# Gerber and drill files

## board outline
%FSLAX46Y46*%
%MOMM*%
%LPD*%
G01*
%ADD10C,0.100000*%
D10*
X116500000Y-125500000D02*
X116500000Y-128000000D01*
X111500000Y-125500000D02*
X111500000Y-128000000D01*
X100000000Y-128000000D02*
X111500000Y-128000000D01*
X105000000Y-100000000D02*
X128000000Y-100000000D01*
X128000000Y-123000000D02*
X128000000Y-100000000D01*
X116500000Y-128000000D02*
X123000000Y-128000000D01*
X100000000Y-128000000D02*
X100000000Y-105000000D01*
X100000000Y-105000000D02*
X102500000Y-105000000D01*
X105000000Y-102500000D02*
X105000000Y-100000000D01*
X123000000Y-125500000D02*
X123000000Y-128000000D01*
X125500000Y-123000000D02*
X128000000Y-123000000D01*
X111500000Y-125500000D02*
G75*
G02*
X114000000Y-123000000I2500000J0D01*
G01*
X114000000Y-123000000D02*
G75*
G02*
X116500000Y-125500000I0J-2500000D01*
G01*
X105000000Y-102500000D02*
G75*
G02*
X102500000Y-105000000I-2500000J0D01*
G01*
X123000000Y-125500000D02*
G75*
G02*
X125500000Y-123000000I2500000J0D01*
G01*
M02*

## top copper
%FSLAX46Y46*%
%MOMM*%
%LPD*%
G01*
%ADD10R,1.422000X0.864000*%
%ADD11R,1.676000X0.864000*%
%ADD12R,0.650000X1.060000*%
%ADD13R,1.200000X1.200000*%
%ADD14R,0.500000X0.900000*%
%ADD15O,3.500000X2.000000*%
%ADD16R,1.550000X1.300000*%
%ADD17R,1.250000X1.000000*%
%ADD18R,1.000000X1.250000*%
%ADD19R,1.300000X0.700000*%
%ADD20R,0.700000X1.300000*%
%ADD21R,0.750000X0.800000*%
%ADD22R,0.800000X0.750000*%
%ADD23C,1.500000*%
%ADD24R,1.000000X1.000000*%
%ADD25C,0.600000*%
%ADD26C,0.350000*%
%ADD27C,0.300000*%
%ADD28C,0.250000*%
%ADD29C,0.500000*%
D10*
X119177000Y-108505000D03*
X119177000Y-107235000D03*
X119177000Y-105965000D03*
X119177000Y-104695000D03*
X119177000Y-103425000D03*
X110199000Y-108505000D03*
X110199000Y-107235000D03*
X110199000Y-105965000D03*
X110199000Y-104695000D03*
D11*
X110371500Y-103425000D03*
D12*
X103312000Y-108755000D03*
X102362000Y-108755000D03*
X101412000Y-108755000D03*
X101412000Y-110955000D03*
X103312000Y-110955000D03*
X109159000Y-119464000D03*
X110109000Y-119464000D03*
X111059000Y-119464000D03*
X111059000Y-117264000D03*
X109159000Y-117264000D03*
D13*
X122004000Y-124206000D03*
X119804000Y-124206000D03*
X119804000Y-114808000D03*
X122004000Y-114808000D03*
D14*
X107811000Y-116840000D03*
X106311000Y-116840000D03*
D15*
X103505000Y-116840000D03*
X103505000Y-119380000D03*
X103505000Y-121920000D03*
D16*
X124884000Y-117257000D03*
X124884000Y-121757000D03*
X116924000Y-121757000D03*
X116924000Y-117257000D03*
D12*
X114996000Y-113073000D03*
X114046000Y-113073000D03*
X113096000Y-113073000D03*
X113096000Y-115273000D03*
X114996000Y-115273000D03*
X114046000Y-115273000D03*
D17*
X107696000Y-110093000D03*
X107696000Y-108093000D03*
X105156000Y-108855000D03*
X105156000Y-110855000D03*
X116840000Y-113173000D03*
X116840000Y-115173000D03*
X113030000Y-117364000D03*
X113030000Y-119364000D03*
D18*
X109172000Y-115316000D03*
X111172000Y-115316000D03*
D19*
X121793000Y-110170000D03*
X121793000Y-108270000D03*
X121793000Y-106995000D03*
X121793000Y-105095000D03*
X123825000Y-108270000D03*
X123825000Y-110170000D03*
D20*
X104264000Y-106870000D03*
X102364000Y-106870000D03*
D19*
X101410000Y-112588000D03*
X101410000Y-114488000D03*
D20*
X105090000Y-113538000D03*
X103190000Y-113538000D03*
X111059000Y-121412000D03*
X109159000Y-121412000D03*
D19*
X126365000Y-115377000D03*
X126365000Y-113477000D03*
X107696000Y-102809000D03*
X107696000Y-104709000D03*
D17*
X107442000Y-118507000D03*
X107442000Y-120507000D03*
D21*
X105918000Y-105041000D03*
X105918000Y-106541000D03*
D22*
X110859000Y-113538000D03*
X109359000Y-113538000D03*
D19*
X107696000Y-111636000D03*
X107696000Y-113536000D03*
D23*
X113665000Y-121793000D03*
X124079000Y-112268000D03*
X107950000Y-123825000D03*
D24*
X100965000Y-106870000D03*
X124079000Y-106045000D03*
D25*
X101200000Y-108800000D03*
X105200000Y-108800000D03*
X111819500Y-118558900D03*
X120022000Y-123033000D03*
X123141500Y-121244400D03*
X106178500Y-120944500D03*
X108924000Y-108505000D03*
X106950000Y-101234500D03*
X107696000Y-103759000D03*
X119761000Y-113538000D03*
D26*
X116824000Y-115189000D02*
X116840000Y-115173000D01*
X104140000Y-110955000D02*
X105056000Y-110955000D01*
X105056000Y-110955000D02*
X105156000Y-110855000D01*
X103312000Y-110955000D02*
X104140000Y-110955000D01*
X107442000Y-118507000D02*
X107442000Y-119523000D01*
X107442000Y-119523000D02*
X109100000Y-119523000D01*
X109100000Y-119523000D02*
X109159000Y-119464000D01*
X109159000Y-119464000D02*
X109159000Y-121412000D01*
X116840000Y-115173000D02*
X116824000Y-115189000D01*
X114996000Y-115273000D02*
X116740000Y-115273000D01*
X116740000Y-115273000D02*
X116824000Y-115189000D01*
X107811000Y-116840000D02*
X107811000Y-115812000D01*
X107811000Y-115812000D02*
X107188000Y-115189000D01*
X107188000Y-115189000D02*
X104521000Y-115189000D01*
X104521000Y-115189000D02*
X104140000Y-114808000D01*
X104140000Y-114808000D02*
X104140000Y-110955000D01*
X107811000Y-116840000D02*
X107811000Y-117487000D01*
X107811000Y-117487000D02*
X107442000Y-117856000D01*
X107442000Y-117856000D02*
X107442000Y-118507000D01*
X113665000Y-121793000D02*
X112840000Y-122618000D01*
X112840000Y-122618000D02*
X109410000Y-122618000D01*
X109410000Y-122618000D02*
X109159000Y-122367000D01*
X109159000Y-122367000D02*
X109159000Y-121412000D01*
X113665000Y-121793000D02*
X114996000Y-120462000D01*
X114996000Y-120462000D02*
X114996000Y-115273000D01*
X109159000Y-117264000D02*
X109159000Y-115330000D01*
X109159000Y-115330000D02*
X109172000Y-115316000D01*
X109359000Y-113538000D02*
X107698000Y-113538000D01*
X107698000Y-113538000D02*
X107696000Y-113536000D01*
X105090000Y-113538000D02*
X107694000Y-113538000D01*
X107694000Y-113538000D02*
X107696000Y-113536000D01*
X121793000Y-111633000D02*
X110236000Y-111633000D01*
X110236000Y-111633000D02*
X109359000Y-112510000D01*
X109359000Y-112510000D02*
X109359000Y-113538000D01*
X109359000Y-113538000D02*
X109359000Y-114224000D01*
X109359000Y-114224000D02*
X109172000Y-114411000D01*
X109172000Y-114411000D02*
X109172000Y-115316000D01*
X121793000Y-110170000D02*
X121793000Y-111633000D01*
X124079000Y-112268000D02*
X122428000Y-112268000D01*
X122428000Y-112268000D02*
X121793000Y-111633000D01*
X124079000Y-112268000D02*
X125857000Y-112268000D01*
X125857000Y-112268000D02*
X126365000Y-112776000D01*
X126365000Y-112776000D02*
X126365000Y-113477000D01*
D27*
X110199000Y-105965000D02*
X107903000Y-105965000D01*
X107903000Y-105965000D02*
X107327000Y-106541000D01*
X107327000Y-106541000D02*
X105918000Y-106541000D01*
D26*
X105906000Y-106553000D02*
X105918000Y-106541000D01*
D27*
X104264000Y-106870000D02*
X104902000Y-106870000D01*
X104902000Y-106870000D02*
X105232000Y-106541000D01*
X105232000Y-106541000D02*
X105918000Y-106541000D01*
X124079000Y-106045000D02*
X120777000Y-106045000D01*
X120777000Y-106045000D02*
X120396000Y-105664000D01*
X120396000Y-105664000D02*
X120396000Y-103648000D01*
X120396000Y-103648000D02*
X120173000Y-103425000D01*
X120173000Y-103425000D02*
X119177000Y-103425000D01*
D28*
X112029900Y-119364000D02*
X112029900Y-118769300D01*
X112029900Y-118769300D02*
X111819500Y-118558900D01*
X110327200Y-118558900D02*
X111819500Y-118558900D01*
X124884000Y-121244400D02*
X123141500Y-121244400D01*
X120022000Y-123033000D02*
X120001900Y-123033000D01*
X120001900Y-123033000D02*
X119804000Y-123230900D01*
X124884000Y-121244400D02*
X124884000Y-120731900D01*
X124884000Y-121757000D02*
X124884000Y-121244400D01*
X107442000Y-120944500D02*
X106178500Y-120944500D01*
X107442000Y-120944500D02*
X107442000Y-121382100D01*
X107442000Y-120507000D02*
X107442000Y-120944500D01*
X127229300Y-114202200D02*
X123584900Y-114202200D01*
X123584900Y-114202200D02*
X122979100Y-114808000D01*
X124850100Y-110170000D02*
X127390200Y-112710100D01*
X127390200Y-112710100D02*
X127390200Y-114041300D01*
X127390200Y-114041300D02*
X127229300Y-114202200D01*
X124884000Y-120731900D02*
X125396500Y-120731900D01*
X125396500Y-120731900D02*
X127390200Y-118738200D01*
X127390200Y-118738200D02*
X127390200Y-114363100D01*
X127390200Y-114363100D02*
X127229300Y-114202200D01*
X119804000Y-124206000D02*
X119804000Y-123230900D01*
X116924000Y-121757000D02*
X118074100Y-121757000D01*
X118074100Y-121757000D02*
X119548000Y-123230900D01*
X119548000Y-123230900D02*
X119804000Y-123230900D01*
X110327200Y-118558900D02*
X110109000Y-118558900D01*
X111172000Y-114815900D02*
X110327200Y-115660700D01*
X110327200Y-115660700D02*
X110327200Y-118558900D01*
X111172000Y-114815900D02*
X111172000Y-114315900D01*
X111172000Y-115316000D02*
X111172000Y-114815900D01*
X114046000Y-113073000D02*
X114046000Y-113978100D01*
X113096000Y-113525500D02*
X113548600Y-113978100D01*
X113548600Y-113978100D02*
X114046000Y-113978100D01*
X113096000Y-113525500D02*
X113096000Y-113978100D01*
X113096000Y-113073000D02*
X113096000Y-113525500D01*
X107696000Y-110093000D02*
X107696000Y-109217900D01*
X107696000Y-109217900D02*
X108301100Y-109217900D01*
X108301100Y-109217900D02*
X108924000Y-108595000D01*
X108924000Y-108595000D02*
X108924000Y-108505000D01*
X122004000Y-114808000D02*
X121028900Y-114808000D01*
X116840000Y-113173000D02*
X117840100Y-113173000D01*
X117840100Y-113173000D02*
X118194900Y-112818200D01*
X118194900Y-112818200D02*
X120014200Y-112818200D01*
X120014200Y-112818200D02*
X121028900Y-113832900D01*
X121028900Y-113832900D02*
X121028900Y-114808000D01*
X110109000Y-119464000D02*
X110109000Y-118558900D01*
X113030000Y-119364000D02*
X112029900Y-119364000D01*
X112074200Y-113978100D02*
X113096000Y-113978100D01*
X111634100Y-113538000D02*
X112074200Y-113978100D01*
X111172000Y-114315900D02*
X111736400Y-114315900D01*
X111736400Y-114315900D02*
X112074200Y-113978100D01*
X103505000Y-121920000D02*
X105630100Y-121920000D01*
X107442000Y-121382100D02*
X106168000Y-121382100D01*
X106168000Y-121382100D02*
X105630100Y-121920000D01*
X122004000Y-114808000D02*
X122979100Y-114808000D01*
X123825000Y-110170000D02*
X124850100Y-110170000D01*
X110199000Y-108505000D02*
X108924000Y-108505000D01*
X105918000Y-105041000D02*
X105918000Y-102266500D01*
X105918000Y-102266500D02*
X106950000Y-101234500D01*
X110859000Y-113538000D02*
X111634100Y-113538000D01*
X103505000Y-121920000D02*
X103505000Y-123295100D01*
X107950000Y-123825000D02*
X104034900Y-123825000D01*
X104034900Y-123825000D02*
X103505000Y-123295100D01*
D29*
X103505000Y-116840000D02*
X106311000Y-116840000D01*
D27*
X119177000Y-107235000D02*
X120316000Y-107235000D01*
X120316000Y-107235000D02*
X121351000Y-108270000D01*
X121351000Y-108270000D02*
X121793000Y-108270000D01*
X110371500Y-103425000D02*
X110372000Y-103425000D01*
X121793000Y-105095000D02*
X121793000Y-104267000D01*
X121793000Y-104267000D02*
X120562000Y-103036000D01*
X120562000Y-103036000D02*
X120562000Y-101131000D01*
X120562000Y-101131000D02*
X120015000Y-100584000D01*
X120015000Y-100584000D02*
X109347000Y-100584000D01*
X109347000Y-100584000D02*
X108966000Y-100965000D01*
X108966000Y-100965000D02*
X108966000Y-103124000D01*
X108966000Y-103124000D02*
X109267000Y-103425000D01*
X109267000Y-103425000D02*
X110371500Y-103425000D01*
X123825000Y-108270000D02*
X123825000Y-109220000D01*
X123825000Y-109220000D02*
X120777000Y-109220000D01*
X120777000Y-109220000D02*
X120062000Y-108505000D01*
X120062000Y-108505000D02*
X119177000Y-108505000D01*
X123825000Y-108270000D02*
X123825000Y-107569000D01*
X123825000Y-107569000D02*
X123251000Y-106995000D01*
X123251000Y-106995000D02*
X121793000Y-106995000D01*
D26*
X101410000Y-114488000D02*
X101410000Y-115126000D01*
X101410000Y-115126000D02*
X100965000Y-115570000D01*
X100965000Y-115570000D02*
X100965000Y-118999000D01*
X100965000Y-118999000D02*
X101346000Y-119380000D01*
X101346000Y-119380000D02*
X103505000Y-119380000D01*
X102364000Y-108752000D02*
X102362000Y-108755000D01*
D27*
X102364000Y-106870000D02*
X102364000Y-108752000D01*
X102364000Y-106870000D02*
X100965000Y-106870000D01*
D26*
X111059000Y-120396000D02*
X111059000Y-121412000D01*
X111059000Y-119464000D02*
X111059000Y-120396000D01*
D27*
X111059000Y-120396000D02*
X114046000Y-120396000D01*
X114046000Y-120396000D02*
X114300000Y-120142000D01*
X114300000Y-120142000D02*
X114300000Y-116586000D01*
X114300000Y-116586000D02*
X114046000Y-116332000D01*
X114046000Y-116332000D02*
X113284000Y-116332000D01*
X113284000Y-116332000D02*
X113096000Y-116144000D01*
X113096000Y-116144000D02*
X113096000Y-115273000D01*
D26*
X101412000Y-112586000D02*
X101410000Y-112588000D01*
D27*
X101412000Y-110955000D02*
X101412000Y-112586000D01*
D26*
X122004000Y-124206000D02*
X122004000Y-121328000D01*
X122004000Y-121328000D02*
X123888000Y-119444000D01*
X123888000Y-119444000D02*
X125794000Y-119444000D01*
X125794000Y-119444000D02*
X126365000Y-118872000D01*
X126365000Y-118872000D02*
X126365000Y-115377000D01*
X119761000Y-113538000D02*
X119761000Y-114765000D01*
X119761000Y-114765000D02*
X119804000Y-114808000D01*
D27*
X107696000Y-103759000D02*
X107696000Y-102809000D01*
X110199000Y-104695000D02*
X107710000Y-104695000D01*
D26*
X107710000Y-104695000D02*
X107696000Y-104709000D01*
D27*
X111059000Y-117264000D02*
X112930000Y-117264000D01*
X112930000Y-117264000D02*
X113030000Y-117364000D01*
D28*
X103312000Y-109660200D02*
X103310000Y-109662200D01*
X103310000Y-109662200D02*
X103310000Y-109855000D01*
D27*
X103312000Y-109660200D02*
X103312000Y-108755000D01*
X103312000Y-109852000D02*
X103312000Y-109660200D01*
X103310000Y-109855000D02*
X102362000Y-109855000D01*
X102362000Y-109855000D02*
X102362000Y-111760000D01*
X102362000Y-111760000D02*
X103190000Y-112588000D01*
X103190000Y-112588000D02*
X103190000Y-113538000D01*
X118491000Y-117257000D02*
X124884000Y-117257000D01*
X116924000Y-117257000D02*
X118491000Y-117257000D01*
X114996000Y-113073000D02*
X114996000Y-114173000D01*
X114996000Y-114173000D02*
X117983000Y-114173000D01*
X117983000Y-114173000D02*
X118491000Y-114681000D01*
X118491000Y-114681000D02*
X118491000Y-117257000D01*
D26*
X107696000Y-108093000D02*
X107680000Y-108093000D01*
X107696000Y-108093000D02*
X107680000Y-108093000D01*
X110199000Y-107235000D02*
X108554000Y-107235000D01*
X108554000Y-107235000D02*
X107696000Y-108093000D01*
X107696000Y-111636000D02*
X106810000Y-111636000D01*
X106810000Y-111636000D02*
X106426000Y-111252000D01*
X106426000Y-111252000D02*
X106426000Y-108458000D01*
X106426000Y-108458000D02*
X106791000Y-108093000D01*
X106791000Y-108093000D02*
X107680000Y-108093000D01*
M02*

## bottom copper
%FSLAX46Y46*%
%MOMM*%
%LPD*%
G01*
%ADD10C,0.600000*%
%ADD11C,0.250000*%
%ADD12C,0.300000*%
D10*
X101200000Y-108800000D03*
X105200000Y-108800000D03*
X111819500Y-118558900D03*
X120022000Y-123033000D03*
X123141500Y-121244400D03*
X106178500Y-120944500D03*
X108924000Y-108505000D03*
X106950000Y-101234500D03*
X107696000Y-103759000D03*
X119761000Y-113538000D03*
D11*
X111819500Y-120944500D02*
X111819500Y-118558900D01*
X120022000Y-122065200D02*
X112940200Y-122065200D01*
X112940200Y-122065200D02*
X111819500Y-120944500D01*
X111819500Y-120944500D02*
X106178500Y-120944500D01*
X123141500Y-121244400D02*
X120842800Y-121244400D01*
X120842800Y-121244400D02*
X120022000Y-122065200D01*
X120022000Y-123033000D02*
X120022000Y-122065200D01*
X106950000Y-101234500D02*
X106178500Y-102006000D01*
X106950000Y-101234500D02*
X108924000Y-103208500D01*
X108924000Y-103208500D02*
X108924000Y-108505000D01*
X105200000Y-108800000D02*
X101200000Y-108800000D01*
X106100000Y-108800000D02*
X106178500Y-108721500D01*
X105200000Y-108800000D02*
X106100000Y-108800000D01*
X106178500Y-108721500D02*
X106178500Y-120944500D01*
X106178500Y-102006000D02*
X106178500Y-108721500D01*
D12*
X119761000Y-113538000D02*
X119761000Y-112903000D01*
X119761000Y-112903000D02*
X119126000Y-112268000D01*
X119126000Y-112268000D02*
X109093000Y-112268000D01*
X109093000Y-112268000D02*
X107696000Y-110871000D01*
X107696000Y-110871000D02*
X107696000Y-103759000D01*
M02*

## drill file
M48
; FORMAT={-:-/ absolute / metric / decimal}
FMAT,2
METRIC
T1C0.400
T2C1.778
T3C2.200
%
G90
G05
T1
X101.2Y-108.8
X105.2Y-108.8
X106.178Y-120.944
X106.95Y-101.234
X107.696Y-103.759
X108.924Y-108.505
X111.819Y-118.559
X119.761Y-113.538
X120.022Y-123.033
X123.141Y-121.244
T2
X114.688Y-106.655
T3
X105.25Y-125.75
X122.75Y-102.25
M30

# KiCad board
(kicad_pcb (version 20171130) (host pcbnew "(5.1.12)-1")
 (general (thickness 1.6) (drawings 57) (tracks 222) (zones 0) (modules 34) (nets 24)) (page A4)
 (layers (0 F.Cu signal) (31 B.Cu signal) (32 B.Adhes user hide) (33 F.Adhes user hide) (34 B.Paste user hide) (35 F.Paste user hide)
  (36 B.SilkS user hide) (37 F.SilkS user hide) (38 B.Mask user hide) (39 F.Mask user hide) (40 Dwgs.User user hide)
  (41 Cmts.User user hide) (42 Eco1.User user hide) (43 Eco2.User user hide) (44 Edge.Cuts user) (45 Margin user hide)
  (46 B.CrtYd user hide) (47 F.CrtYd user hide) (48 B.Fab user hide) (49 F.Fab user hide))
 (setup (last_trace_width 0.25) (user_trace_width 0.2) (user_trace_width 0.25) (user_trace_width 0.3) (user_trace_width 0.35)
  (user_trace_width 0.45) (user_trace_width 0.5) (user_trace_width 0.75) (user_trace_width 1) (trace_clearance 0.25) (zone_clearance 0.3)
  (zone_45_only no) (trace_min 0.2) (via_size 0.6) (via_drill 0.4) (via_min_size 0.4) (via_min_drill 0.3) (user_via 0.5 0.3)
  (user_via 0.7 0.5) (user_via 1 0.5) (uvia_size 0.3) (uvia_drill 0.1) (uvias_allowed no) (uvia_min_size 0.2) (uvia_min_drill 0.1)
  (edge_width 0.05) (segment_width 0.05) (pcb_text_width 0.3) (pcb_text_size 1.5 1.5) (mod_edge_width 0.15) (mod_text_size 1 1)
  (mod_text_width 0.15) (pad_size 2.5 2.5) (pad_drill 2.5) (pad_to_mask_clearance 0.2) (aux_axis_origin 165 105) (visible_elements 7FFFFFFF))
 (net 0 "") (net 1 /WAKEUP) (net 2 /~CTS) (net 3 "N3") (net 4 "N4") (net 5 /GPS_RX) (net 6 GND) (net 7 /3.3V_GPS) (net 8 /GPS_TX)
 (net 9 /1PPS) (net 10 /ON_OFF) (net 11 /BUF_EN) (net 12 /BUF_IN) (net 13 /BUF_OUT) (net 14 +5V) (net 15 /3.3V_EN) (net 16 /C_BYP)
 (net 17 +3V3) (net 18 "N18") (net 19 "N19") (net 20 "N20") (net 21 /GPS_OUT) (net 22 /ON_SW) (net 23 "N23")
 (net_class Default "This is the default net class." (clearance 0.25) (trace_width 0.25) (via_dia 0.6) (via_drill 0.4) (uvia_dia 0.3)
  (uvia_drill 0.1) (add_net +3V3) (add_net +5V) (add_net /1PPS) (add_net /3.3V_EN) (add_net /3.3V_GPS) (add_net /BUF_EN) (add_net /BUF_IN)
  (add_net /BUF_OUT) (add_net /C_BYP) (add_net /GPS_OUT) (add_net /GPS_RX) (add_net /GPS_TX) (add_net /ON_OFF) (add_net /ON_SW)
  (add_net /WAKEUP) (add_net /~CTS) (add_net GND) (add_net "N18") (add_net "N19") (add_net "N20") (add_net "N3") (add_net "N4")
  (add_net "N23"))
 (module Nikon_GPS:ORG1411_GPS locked (layer F.Cu) (at 119.888 100.965 180)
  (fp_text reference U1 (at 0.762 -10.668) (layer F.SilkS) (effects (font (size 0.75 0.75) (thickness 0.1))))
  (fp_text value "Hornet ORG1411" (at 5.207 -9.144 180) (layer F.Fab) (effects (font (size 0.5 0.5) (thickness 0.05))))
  (pad 6 smd rect (at 0.711 -7.54 180) (size 1.422 0.864) (layers F.Cu F.Paste F.Mask) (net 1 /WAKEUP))
  (pad 7 smd rect (at 0.711 -6.27 180) (size 1.422 0.864) (layers F.Cu F.Paste F.Mask) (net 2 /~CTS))
  (pad 8 smd rect (at 0.711 -5 180) (size 1.422 0.864) (layers F.Cu F.Paste F.Mask) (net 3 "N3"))
  (pad 9 smd rect (at 0.711 -3.73 180) (size 1.422 0.864) (layers F.Cu F.Paste F.Mask) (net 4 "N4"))
  (pad 10 smd rect (at 0.711 -2.46 180) (size 1.422 0.864) (layers F.Cu F.Paste F.Mask) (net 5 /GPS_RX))
  (pad 5 smd rect (at 9.689 -7.54 180) (size 1.422 0.864) (layers F.Cu F.Paste F.Mask) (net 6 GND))
  (pad 4 smd rect (at 9.689 -6.27 180) (size 1.422 0.864) (layers F.Cu F.Paste F.Mask) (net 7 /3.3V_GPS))
  (pad 3 smd rect (at 9.689 -5 180) (size 1.422 0.864) (layers F.Cu F.Paste F.Mask) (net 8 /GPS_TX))
  (pad 2 smd rect (at 9.689 -3.73 180) (size 1.422 0.864) (layers F.Cu F.Paste F.Mask) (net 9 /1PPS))
  (pad "" np_thru_hole circle (at 5.2 -5.69 180) (size 1.778 1.778) (drill 1.778) (layers *.Cu *.Mask))
  (pad 1 smd rect (at 9.5165 -2.46 180) (size 1.676 0.864) (layers F.Cu F.Paste F.Mask) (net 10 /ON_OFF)))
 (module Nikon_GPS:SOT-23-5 (layer F.Cu) (at 102.362 109.855 270)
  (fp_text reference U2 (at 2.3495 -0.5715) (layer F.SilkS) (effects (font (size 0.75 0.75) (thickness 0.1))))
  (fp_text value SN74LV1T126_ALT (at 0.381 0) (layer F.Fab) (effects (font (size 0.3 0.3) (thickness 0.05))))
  (pad 1 smd rect (at -1.1 -0.95 270) (size 1.06 0.65) (layers F.Cu F.Paste F.Mask) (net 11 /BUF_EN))
  (pad 2 smd rect (at -1.1 0 270) (size 1.06 0.65) (layers F.Cu F.Paste F.Mask) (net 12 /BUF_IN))
  (pad 3 smd rect (at -1.1 0.95 270) (size 1.06 0.65) (layers F.Cu F.Paste F.Mask) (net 6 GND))
  (pad 4 smd rect (at 1.1 0.95 270) (size 1.06 0.65) (layers F.Cu F.Paste F.Mask) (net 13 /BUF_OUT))
  (pad 5 smd rect (at 1.1 -0.95 270) (size 1.06 0.65) (layers F.Cu F.Paste F.Mask) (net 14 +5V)))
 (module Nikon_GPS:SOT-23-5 (layer F.Cu) (at 110.109 118.364 90)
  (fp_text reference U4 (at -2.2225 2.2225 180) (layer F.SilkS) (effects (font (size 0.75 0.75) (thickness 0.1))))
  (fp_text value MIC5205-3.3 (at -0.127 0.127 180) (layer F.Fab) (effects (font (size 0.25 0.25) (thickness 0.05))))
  (pad 1 smd rect (at -1.1 -0.95 90) (size 1.06 0.65) (layers F.Cu F.Paste F.Mask) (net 14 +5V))
  (pad 2 smd rect (at -1.1 0 90) (size 1.06 0.65) (layers F.Cu F.Paste F.Mask) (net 6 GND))
  (pad 3 smd rect (at -1.1 0.95 90) (size 1.06 0.65) (layers F.Cu F.Paste F.Mask) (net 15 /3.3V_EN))
  (pad 4 smd rect (at 1.1 0.95 90) (size 1.06 0.65) (layers F.Cu F.Paste F.Mask) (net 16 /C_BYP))
  (pad 5 smd rect (at 1.1 -0.95 90) (size 1.06 0.65) (layers F.Cu F.Paste F.Mask) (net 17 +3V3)))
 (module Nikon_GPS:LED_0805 (layer F.Cu) (at 120.904 124.206)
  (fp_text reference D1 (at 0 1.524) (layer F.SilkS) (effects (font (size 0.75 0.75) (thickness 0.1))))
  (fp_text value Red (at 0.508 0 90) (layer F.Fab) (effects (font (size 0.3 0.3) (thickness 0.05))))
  (pad 2 smd rect (at 1.1 0 180) (size 1.2 1.2) (layers F.Cu F.Paste F.Mask) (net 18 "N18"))
  (pad 1 smd rect (at -1.1 0 180) (size 1.2 1.2) (layers F.Cu F.Paste F.Mask) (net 6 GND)))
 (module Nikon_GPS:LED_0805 (layer F.Cu) (at 120.904 114.808 180)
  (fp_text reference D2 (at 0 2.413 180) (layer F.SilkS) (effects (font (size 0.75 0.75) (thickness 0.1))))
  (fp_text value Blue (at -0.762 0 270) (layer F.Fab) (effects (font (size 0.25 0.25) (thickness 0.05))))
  (pad 2 smd rect (at 1.1 0) (size 1.2 1.2) (layers F.Cu F.Paste F.Mask) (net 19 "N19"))
  (pad 1 smd rect (at -1.1 0) (size 1.2 1.2) (layers F.Cu F.Paste F.Mask) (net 6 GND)))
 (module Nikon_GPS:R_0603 (layer F.Cu) (at 107.061 116.84 180)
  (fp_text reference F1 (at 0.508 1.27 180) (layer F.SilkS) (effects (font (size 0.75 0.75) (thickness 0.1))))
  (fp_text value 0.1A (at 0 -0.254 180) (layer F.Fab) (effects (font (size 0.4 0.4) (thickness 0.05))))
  (pad 1 smd rect (at -0.75 0 180) (size 0.5 0.9) (layers F.Cu F.Paste F.Mask) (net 14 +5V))
  (pad 2 smd rect (at 0.75 0 180) (size 0.5 0.9) (layers F.Cu F.Paste F.Mask) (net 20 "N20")))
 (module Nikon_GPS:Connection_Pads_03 (layer F.Cu) (at 103.505 119.38 270)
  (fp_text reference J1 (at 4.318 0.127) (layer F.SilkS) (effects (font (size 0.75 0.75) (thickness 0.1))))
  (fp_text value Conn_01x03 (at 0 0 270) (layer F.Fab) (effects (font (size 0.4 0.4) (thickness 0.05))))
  (pad 1 smd oval (at -2.54 0 270) (size 2 3.5) (layers F.Cu F.Paste F.Mask) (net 20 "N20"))
  (pad 2 smd oval (at 0 0 270) (size 2 3.5) (layers F.Cu F.Paste F.Mask) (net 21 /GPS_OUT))
  (pad 3 smd oval (at 2.54 0 270) (size 2 3.5) (layers F.Cu F.Paste F.Mask) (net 6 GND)))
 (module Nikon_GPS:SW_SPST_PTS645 (layer F.Cu) (at 120.904 119.507 180)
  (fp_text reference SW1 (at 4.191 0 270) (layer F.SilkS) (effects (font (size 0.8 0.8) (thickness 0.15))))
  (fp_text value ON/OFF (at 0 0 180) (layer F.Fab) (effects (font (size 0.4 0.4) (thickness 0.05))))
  (pad 2 smd rect (at -3.98 2.25 180) (size 1.55 1.3) (layers F.Cu F.Paste F.Mask) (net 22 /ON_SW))
  (pad 1 smd rect (at -3.98 -2.25 180) (size 1.55 1.3) (layers F.Cu F.Paste F.Mask) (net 6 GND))
  (pad 1 smd rect (at 3.98 -2.25 180) (size 1.55 1.3) (layers F.Cu F.Paste F.Mask) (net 6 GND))
  (pad 2 smd rect (at 3.98 2.25 180) (size 1.55 1.3) (layers F.Cu F.Paste F.Mask) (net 22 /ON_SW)))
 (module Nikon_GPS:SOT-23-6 (layer F.Cu) (at 114.046 114.173 270)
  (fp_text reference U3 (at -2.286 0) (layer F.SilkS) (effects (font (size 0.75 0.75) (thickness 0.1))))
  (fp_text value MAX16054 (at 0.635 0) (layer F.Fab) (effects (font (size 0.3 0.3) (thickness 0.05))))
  (pad 1 smd rect (at -1.1 -0.95 270) (size 1.06 0.65) (layers F.Cu F.Paste F.Mask) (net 22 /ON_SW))
  (pad 2 smd rect (at -1.1 0 270) (size 1.06 0.65) (layers F.Cu F.Paste F.Mask) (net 6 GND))
  (pad 3 smd rect (at -1.1 0.95 270) (size 1.06 0.65) (layers F.Cu F.Paste F.Mask) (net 6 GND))
  (pad 4 smd rect (at 1.1 0.95 270) (size 1.06 0.65) (layers F.Cu F.Paste F.Mask) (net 15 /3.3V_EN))
  (pad 6 smd rect (at 1.1 -0.95 270) (size 1.06 0.65) (layers F.Cu F.Paste F.Mask) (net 14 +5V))
  (pad 5 smd rect (at 1.1 0 270) (size 1.06 0.65) (layers F.Cu F.Paste F.Mask) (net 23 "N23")))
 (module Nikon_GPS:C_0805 (layer F.Cu) (at 107.696 109.093 90)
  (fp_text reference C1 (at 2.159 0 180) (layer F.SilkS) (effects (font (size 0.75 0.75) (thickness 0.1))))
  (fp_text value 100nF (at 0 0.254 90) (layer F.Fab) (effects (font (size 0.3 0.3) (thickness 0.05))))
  (pad 1 smd rect (at -1 0 90) (size 1 1.25) (layers F.Cu F.Paste F.Mask) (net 6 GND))
  (pad 2 smd rect (at 1 0 90) (size 1 1.25) (layers F.Cu F.Paste F.Mask) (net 7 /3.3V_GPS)))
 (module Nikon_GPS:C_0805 (layer F.Cu) (at 105.156 109.855 270)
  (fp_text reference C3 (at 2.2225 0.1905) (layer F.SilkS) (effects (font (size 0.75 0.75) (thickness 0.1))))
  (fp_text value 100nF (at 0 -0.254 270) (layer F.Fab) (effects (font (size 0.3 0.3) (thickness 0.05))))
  (pad 1 smd rect (at -1 0 270) (size 1 1.25) (layers F.Cu F.Paste F.Mask) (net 6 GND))
  (pad 2 smd rect (at 1 0 270) (size 1 1.25) (layers F.Cu F.Paste F.Mask) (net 14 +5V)))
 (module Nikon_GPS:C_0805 (layer F.Cu) (at 116.84 114.173 270)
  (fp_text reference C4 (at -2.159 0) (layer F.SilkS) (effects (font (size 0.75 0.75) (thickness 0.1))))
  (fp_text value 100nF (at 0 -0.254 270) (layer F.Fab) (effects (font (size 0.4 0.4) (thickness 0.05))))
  (pad 1 smd rect (at -1 0 270) (size 1 1.25) (layers F.Cu F.Paste F.Mask) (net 6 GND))
  (pad 2 smd rect (at 1 0 270) (size 1 1.25) (layers F.Cu F.Paste F.Mask) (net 14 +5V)))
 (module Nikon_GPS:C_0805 (layer F.Cu) (at 113.03 118.364 270)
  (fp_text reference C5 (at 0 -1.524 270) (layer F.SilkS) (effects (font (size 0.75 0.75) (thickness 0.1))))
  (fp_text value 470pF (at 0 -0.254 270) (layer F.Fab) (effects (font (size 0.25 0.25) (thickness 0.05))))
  (pad 1 smd rect (at -1 0 270) (size 1 1.25) (layers F.Cu F.Paste F.Mask) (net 16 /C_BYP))
  (pad 2 smd rect (at 1 0 270) (size 1 1.25) (layers F.Cu F.Paste F.Mask) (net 6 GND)))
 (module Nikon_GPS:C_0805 (layer F.Cu) (at 110.172 115.316)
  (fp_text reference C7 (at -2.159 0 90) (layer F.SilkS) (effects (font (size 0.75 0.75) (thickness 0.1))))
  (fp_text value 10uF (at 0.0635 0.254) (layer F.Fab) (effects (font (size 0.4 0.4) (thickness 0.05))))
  (pad 1 smd rect (at -1 0) (size 1 1.25) (layers F.Cu F.Paste F.Mask) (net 17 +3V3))
  (pad 2 smd rect (at 1 0) (size 1 1.25) (layers F.Cu F.Paste F.Mask) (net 6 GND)))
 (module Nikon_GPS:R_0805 (layer F.Cu) (at 121.793 109.22 90)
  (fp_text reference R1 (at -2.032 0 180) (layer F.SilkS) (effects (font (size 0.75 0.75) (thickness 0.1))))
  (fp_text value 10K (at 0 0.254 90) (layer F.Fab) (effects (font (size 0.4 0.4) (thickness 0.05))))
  (pad 1 smd rect (at -0.95 0 90) (size 0.7 1.3) (layers F.Cu F.Paste F.Mask) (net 17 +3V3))
  (pad 2 smd rect (at 0.95 0 90) (size 0.7 1.3) (layers F.Cu F.Paste F.Mask) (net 2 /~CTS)))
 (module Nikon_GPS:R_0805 (layer F.Cu) (at 121.793 106.045 90)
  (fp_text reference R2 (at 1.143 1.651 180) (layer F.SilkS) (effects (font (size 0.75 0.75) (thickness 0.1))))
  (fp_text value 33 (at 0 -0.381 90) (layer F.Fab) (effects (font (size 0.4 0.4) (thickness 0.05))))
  (pad 1 smd rect (at -0.95 0 90) (size 0.7 1.3) (layers F.Cu F.Paste F.Mask) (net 1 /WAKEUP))
  (pad 2 smd rect (at 0.95 0 90) (size 0.7 1.3) (layers F.Cu F.Paste F.Mask) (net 10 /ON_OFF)))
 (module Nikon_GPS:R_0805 (layer F.Cu) (at 123.825 109.22 270)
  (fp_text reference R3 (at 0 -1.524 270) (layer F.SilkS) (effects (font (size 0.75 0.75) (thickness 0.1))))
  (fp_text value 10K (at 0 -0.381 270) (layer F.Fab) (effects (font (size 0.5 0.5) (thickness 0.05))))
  (pad 1 smd rect (at -0.95 0 270) (size 0.7 1.3) (layers F.Cu F.Paste F.Mask) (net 1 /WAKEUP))
  (pad 2 smd rect (at 0.95 0 270) (size 0.7 1.3) (layers F.Cu F.Paste F.Mask) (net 6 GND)))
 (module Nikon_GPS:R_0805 (layer F.Cu) (at 103.314 106.87 180)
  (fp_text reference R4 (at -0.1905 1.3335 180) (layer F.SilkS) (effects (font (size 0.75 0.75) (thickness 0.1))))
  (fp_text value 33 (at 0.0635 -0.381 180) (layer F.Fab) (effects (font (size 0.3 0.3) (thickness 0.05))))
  (pad 1 smd rect (at -0.95 0 180) (size 0.7 1.3) (layers F.Cu F.Paste F.Mask) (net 8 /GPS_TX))
  (pad 2 smd rect (at 0.95 0 180) (size 0.7 1.3) (layers F.Cu F.Paste F.Mask) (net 12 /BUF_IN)))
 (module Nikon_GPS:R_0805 (layer F.Cu) (at 101.41 113.538 270)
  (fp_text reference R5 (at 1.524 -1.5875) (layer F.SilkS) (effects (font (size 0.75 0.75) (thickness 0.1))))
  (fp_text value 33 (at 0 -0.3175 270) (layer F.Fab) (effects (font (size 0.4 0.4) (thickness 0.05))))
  (pad 1 smd rect (at -0.95 0 270) (size 0.7 1.3) (layers F.Cu F.Paste F.Mask) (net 13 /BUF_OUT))
  (pad 2 smd rect (at 0.95 0 270) (size 0.7 1.3) (layers F.Cu F.Paste F.Mask) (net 21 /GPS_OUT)))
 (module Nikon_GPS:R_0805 (layer F.Cu) (at 104.14 113.538 180)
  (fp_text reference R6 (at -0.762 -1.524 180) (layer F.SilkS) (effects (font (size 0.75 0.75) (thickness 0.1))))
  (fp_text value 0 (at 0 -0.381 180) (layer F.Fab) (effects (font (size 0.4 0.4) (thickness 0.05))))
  (pad 1 smd rect (at -0.95 0 180) (size 0.7 1.3) (layers F.Cu F.Paste F.Mask) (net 17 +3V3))
  (pad 2 smd rect (at 0.95 0 180) (size 0.7 1.3) (layers F.Cu F.Paste F.Mask) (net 11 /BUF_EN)))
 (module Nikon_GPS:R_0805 (layer F.Cu) (at 110.109 121.412 180)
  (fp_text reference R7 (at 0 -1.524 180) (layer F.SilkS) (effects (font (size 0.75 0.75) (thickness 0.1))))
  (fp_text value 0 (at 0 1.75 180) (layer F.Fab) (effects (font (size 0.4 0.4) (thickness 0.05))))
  (pad 1 smd rect (at -0.95 0 180) (size 0.7 1.3) (layers F.Cu F.Paste F.Mask) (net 15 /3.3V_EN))
  (pad 2 smd rect (at 0.95 0 180) (size 0.7 1.3) (layers F.Cu F.Paste F.Mask) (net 14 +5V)))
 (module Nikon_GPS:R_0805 (layer F.Cu) (at 126.365 114.427 90)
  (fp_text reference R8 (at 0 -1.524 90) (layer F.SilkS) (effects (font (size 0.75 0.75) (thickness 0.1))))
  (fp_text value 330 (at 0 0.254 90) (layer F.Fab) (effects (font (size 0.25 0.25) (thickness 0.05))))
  (pad 1 smd rect (at -0.95 0 90) (size 0.7 1.3) (layers F.Cu F.Paste F.Mask) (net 18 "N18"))
  (pad 2 smd rect (at 0.95 0 90) (size 0.7 1.3) (layers F.Cu F.Paste F.Mask) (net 17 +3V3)))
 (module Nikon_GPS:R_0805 (layer F.Cu) (at 107.696 103.759 270)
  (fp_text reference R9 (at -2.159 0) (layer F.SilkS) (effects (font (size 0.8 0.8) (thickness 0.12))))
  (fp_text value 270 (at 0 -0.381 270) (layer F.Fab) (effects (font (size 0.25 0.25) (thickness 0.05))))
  (pad 1 smd rect (at -0.95 0 270) (size 0.7 1.3) (layers F.Cu F.Paste F.Mask) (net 19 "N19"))
  (pad 2 smd rect (at 0.95 0 270) (size 0.7 1.3) (layers F.Cu F.Paste F.Mask) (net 9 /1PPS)))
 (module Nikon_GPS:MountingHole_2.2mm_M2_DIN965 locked (layer F.Cu) (at 105.25 125.75)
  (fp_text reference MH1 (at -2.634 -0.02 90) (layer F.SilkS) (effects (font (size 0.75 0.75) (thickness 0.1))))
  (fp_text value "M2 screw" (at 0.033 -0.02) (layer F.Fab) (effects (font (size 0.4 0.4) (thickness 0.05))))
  (pad 1 np_thru_hole circle (at 0 0) (size 2.2 2.2) (drill 2.2) (layers *.Cu *.Mask)))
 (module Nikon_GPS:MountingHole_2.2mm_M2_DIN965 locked (layer F.Cu) (at 122.75 102.25)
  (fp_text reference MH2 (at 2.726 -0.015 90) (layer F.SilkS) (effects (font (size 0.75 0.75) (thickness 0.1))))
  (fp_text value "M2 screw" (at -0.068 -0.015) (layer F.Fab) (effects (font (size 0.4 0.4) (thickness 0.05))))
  (pad 1 np_thru_hole circle (at 0 0) (size 2.2 2.2) (drill 2.2) (layers *.Cu *.Mask)))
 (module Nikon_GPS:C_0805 (layer F.Cu) (at 107.442 119.507 270)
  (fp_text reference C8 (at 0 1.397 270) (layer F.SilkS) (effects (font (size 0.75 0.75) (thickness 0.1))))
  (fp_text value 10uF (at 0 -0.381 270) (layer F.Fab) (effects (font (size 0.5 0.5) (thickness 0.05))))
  (pad 1 smd rect (at -1 0 270) (size 1 1.25) (layers F.Cu F.Paste F.Mask) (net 14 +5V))
  (pad 2 smd rect (at 1 0 270) (size 1 1.25) (layers F.Cu F.Paste F.Mask) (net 6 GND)))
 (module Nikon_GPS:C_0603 (layer F.Cu) (at 105.918 105.791 90)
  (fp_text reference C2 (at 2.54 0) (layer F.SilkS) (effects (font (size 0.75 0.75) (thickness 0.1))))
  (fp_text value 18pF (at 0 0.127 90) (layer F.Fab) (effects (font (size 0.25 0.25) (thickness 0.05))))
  (pad 2 smd rect (at 0.75 0 90) (size 0.8 0.75) (layers F.Cu F.Paste F.Mask) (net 6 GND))
  (pad 1 smd rect (at -0.75 0 90) (size 0.8 0.75) (layers F.Cu F.Paste F.Mask) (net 8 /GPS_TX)))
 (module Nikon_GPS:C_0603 (layer F.Cu) (at 110.109 113.538)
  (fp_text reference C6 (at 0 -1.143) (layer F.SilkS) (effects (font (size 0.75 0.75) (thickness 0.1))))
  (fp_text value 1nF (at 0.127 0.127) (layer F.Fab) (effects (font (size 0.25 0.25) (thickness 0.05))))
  (pad 2 smd rect (at 0.75 0) (size 0.8 0.75) (layers F.Cu F.Paste F.Mask) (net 6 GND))
  (pad 1 smd rect (at -0.75 0) (size 0.8 0.75) (layers F.Cu F.Paste F.Mask) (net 17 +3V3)))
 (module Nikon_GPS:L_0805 (layer F.Cu) (at 107.696 112.586 270)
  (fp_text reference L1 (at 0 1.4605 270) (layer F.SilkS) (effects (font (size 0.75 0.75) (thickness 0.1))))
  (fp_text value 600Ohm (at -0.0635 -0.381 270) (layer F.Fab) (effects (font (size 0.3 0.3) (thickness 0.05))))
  (pad 1 smd rect (at -0.95 0 270) (size 0.7 1.3) (layers F.Cu F.Paste F.Mask) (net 7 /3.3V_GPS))
  (pad 2 smd rect (at 0.95 0 270) (size 0.7 1.3) (layers F.Cu F.Paste F.Mask) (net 17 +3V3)))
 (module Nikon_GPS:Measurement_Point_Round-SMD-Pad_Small (layer F.Cu) (at 113.665 121.793)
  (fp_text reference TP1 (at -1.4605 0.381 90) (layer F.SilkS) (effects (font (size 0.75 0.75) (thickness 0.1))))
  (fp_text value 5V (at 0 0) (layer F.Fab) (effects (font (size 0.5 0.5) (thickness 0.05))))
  (pad 1 smd circle (at 0 0) (size 1.5 1.5) (layers F.Cu F.Mask) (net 14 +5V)))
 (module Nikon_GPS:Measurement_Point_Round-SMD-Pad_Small (layer F.Cu) (at 124.079 112.268)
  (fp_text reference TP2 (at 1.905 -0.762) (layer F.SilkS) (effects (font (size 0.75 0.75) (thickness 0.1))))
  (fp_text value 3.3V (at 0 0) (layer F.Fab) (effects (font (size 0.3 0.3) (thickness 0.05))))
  (pad 1 smd circle (at 0 0) (size 1.5 1.5) (layers F.Cu F.Mask) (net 17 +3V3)))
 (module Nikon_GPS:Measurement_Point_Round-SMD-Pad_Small (layer F.Cu) (at 107.95 123.825)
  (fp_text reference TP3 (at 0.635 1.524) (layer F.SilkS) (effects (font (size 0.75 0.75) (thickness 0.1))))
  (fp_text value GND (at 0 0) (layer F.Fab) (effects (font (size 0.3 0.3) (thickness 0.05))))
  (pad 1 smd circle (at 0 0) (size 1.5 1.5) (layers F.Cu F.Mask) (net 6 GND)))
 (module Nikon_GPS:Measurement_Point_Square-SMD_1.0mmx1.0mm (layer F.Cu) (at 100.965 106.87)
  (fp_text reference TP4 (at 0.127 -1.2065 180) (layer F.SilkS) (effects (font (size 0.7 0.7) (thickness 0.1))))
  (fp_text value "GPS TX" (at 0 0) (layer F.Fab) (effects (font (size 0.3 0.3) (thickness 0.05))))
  (pad 1 smd rect (at 0 0) (size 1 1) (layers F.Cu F.Mask) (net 12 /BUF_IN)))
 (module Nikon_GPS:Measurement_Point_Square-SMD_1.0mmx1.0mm (layer F.Cu) (at 124.079 106.045)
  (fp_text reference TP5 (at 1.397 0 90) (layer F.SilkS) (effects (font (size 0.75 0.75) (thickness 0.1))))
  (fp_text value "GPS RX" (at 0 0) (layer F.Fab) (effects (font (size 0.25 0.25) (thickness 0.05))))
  (pad 1 smd rect (at 0 0) (size 1 1) (layers F.Cu F.Mask) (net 5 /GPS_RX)))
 (gr_line (start 116.5 125.5) (end 116.5 128) (angle 90) (layer Edge.Cuts) (width 0.1))
 (gr_line (start 111.5 125.5) (end 111.5 128) (angle 90) (layer Edge.Cuts) (width 0.1))
 (gr_line (start 100 128) (end 111.5 128) (layer Edge.Cuts) (width 0.1))
 (gr_line (start 105 100) (end 128 100) (layer Edge.Cuts) (width 0.1))
 (gr_line (start 128 123) (end 128 100) (layer Edge.Cuts) (width 0.1))
 (gr_line (start 116.5 128) (end 123 128) (layer Edge.Cuts) (width 0.1))
 (gr_line (start 100 128) (end 100 105) (layer Edge.Cuts) (width 0.1))
 (gr_line (start 100 105) (end 102.5 105) (layer Edge.Cuts) (width 0.1))
 (gr_line (start 105 102.5) (end 105 100) (layer Edge.Cuts) (width 0.1))
 (gr_line (start 123 125.5) (end 123 128) (layer Edge.Cuts) (width 0.1))
 (gr_line (start 125.5 123) (end 128 123) (layer Edge.Cuts) (width 0.1))
 (gr_arc (start 114 125.5) (end 111.5 125.5) (angle 90) (layer Edge.Cuts) (width 0.1))
 (gr_arc (start 114 125.5) (end 114 123) (angle 90) (layer Edge.Cuts) (width 0.1))
 (gr_arc (start 102.5 102.5) (end 102.5 105) (angle -90) (layer Edge.Cuts) (width 0.1))
 (gr_arc (start 125.5 125.5) (end 125.5 123) (angle -90) (layer Edge.Cuts) (width 0.1))
 (via (at 101.2 108.8) (size 0.6) (drill 0.4) (layers F.Cu B.Cu) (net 6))
 (via (at 105.2 108.8) (size 0.6) (drill 0.4) (layers F.Cu B.Cu) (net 6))
 (segment (start 116.824 115.189) (end 116.84 115.173) (width 0.35) (layer F.Cu) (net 14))
 (segment (start 104.14 110.955) (end 105.056 110.955) (width 0.35) (layer F.Cu) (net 14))
 (segment (start 105.056 110.955) (end 105.156 110.855) (width 0.35) (layer F.Cu) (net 14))
 (segment (start 103.312 110.955) (end 104.14 110.955) (width 0.35) (layer F.Cu) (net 14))
 (segment (start 107.442 118.507) (end 107.442 119.523) (width 0.35) (layer F.Cu) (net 14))
 (segment (start 107.442 119.523) (end 109.1 119.523) (width 0.35) (layer F.Cu) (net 14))
 (segment (start 109.1 119.523) (end 109.159 119.464) (width 0.35) (layer F.Cu) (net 14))
 (segment (start 109.159 119.464) (end 109.159 121.412) (width 0.35) (layer F.Cu) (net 14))
 (segment (start 116.84 115.173) (end 116.824 115.189) (width 0.35) (layer F.Cu) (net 14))
 (segment (start 114.996 115.273) (end 116.74 115.273) (width 0.35) (layer F.Cu) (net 14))
 (segment (start 116.74 115.273) (end 116.824 115.189) (width 0.35) (layer F.Cu) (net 14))
 (segment (start 107.811 116.84) (end 107.811 115.812) (width 0.35) (layer F.Cu) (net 14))
 (segment (start 107.811 115.812) (end 107.188 115.189) (width 0.35) (layer F.Cu) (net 14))
 (segment (start 107.188 115.189) (end 104.521 115.189) (width 0.35) (layer F.Cu) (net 14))
 (segment (start 104.521 115.189) (end 104.14 114.808) (width 0.35) (layer F.Cu) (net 14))
 (segment (start 104.14 114.808) (end 104.14 110.955) (width 0.35) (layer F.Cu) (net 14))
 (segment (start 107.811 116.84) (end 107.811 117.487) (width 0.35) (layer F.Cu) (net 14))
 (segment (start 107.811 117.487) (end 107.442 117.856) (width 0.35) (layer F.Cu) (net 14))
 (segment (start 107.442 117.856) (end 107.442 118.507) (width 0.35) (layer F.Cu) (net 14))
 (segment (start 113.665 121.793) (end 112.84 122.618) (width 0.35) (layer F.Cu) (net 14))
 (segment (start 112.84 122.618) (end 109.41 122.618) (width 0.35) (layer F.Cu) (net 14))
 (segment (start 109.41 122.618) (end 109.159 122.367) (width 0.35) (layer F.Cu) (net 14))
 (segment (start 109.159 122.367) (end 109.159 121.412) (width 0.35) (layer F.Cu) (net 14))
 (segment (start 113.665 121.793) (end 114.996 120.462) (width 0.35) (layer F.Cu) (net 14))
 (segment (start 114.996 120.462) (end 114.996 115.273) (width 0.35) (layer F.Cu) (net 14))
 (segment (start 109.159 117.264) (end 109.159 115.33) (width 0.35) (layer F.Cu) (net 17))
 (segment (start 109.159 115.33) (end 109.172 115.316) (width 0.35) (layer F.Cu) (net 17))
 (segment (start 109.359 113.538) (end 107.698 113.538) (width 0.35) (layer F.Cu) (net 17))
 (segment (start 107.698 113.538) (end 107.696 113.536) (width 0.35) (layer F.Cu) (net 17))
 (segment (start 105.09 113.538) (end 107.694 113.538) (width 0.35) (layer F.Cu) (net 17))
 (segment (start 107.694 113.538) (end 107.696 113.536) (width 0.35) (layer F.Cu) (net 17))
 (segment (start 121.793 111.633) (end 110.236 111.633) (width 0.35) (layer F.Cu) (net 17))
 (segment (start 110.236 111.633) (end 109.359 112.51) (width 0.35) (layer F.Cu) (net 17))
 (segment (start 109.359 112.51) (end 109.359 113.538) (width 0.35) (layer F.Cu) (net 17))
 (segment (start 109.359 113.538) (end 109.359 114.224) (width 0.35) (layer F.Cu) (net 17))
 (segment (start 109.359 114.224) (end 109.172 114.411) (width 0.35) (layer F.Cu) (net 17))
 (segment (start 109.172 114.411) (end 109.172 115.316) (width 0.35) (layer F.Cu) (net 17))
 (segment (start 121.793 110.17) (end 121.793 111.633) (width 0.35) (layer F.Cu) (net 17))
 (segment (start 124.079 112.268) (end 122.428 112.268) (width 0.35) (layer F.Cu) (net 17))
 (segment (start 122.428 112.268) (end 121.793 111.633) (width 0.35) (layer F.Cu) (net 17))
 (segment (start 124.079 112.268) (end 125.857 112.268) (width 0.35) (layer F.Cu) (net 17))
 (segment (start 125.857 112.268) (end 126.365 112.776) (width 0.35) (layer F.Cu) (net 17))
 (segment (start 126.365 112.776) (end 126.365 113.477) (width 0.35) (layer F.Cu) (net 17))
 (segment (start 110.199 105.965) (end 107.903 105.965) (width 0.3) (layer F.Cu) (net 8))
 (segment (start 107.903 105.965) (end 107.327 106.541) (width 0.3) (layer F.Cu) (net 8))
 (segment (start 107.327 106.541) (end 105.918 106.541) (width 0.3) (layer F.Cu) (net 8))
 (segment (start 105.906 106.553) (end 105.918 106.541) (width 0.35) (layer F.Cu) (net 8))
 (segment (start 104.264 106.87) (end 104.902 106.87) (width 0.3) (layer F.Cu) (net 8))
 (segment (start 104.902 106.87) (end 105.232 106.541) (width 0.3) (layer F.Cu) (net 8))
 (segment (start 105.232 106.541) (end 105.918 106.541) (width 0.3) (layer F.Cu) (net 8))
 (segment (start 124.079 106.045) (end 120.777 106.045) (width 0.3) (layer F.Cu) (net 5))
 (segment (start 120.777 106.045) (end 120.396 105.664) (width 0.3) (layer F.Cu) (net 5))
 (segment (start 120.396 105.664) (end 120.396 103.648) (width 0.3) (layer F.Cu) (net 5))
 (segment (start 120.396 103.648) (end 120.173 103.425) (width 0.3) (layer F.Cu) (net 5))
 (segment (start 120.173 103.425) (end 119.177 103.425) (width 0.3) (layer F.Cu) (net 5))
 (segment (start 111.8195 120.9445) (end 111.8195 118.5589) (width 0.25) (layer B.Cu) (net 6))
 (segment (start 120.022 122.0652) (end 112.9402 122.0652) (width 0.25) (layer B.Cu) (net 6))
 (segment (start 112.9402 122.0652) (end 111.8195 120.9445) (width 0.25) (layer B.Cu) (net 6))
 (segment (start 111.8195 120.9445) (end 106.1785 120.9445) (width 0.25) (layer B.Cu) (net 6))
 (segment (start 112.0299 119.364) (end 112.0299 118.7693) (width 0.25) (layer F.Cu) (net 6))
 (segment (start 112.0299 118.7693) (end 111.8195 118.5589) (width 0.25) (layer F.Cu) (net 6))
 (segment (start 110.3272 118.5589) (end 111.8195 118.5589) (width 0.25) (layer F.Cu) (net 6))
 (segment (start 123.1415 121.2444) (end 120.8428 121.2444) (width 0.25) (layer B.Cu) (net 6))
 (segment (start 120.8428 121.2444) (end 120.022 122.0652) (width 0.25) (layer B.Cu) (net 6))
 (segment (start 120.022 123.033) (end 120.022 122.0652) (width 0.25) (layer B.Cu) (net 6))
 (segment (start 124.884 121.2444) (end 123.1415 121.2444) (width 0.25) (layer F.Cu) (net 6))
 (segment (start 120.022 123.033) (end 120.0019 123.033) (width 0.25) (layer F.Cu) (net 6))
 (segment (start 120.0019 123.033) (end 119.804 123.2309) (width 0.25) (layer F.Cu) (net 6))
 (segment (start 124.884 121.2444) (end 124.884 120.7319) (width 0.25) (layer F.Cu) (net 6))
 (segment (start 124.884 121.757) (end 124.884 121.2444) (width 0.25) (layer F.Cu) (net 6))
 (segment (start 107.442 120.9445) (end 106.1785 120.9445) (width 0.25) (layer F.Cu) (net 6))
 (segment (start 106.95 101.2345) (end 106.1785 102.006) (width 0.25) (layer B.Cu) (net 6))
 (segment (start 107.442 120.9445) (end 107.442 121.3821) (width 0.25) (layer F.Cu) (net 6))
 (segment (start 107.442 120.507) (end 107.442 120.9445) (width 0.25) (layer F.Cu) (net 6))
 (segment (start 127.2293 114.2022) (end 123.5849 114.2022) (width 0.25) (layer F.Cu) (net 6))
 (segment (start 123.5849 114.2022) (end 122.9791 114.808) (width 0.25) (layer F.Cu) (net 6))
 (segment (start 124.8501 110.17) (end 127.3902 112.7101) (width 0.25) (layer F.Cu) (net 6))
 (segment (start 127.3902 112.7101) (end 127.3902 114.0413) (width 0.25) (layer F.Cu) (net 6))
 (segment (start 127.3902 114.0413) (end 127.2293 114.2022) (width 0.25) (layer F.Cu) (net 6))
 (segment (start 124.884 120.7319) (end 125.3965 120.7319) (width 0.25) (layer F.Cu) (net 6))
 (segment (start 125.3965 120.7319) (end 127.3902 118.7382) (width 0.25) (layer F.Cu) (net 6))
 (segment (start 127.3902 118.7382) (end 127.3902 114.3631) (width 0.25) (layer F.Cu) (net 6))
 (segment (start 127.3902 114.3631) (end 127.2293 114.2022) (width 0.25) (layer F.Cu) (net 6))
 (segment (start 119.804 124.206) (end 119.804 123.2309) (width 0.25) (layer F.Cu) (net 6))
 (segment (start 116.924 121.757) (end 118.0741 121.757) (width 0.25) (layer F.Cu) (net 6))
 (segment (start 118.0741 121.757) (end 119.548 123.2309) (width 0.25) (layer F.Cu) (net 6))
 (segment (start 119.548 123.2309) (end 119.804 123.2309) (width 0.25) (layer F.Cu) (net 6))
 (segment (start 110.3272 118.5589) (end 110.109 118.5589) (width 0.25) (layer F.Cu) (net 6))
 (segment (start 111.172 114.8159) (end 110.3272 115.6607) (width 0.25) (layer F.Cu) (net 6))
 (segment (start 110.3272 115.6607) (end 110.3272 118.5589) (width 0.25) (layer F.Cu) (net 6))
 (segment (start 111.172 114.8159) (end 111.172 114.3159) (width 0.25) (layer F.Cu) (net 6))
 (segment (start 111.172 115.316) (end 111.172 114.8159) (width 0.25) (layer F.Cu) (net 6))
 (segment (start 114.046 113.073) (end 114.046 113.9781) (width 0.25) (layer F.Cu) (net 6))
 (segment (start 113.096 113.5255) (end 113.5486 113.9781) (width 0.25) (layer F.Cu) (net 6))
 (segment (start 113.5486 113.9781) (end 114.046 113.9781) (width 0.25) (layer F.Cu) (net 6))
 (segment (start 113.096 113.5255) (end 113.096 113.9781) (width 0.25) (layer F.Cu) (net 6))
 (segment (start 113.096 113.073) (end 113.096 113.5255) (width 0.25) (layer F.Cu) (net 6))
 (segment (start 107.696 110.093) (end 107.696 109.2179) (width 0.25) (layer F.Cu) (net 6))
 (segment (start 107.696 109.2179) (end 108.3011 109.2179) (width 0.25) (layer F.Cu) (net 6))
 (segment (start 108.3011 109.2179) (end 108.924 108.595) (width 0.25) (layer F.Cu) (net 6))
 (segment (start 108.924 108.595) (end 108.924 108.505) (width 0.25) (layer F.Cu) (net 6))
 (segment (start 122.004 114.808) (end 121.0289 114.808) (width 0.25) (layer F.Cu) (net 6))
 (segment (start 116.84 113.173) (end 117.8401 113.173) (width 0.25) (layer F.Cu) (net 6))
 (segment (start 117.8401 113.173) (end 118.1949 112.8182) (width 0.25) (layer F.Cu) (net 6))
 (segment (start 118.1949 112.8182) (end 120.0142 112.8182) (width 0.25) (layer F.Cu) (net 6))
 (segment (start 120.0142 112.8182) (end 121.0289 113.8329) (width 0.25) (layer F.Cu) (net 6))
 (segment (start 121.0289 113.8329) (end 121.0289 114.808) (width 0.25) (layer F.Cu) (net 6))
 (segment (start 110.109 119.464) (end 110.109 118.5589) (width 0.25) (layer F.Cu) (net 6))
 (segment (start 113.03 119.364) (end 112.0299 119.364) (width 0.25) (layer F.Cu) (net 6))
 (segment (start 112.0742 113.9781) (end 113.096 113.9781) (width 0.25) (layer F.Cu) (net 6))
 (segment (start 111.6341 113.538) (end 112.0742 113.9781) (width 0.25) (layer F.Cu) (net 6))
 (segment (start 111.172 114.3159) (end 111.7364 114.3159) (width 0.25) (layer F.Cu) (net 6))
 (segment (start 111.7364 114.3159) (end 112.0742 113.9781) (width 0.25) (layer F.Cu) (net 6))
 (segment (start 103.505 121.92) (end 105.6301 121.92) (width 0.25) (layer F.Cu) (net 6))
 (segment (start 107.442 121.3821) (end 106.168 121.3821) (width 0.25) (layer F.Cu) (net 6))
 (segment (start 106.168 121.3821) (end 105.6301 121.92) (width 0.25) (layer F.Cu) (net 6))
 (segment (start 122.004 114.808) (end 122.9791 114.808) (width 0.25) (layer F.Cu) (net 6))
 (segment (start 123.825 110.17) (end 124.8501 110.17) (width 0.25) (layer F.Cu) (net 6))
 (segment (start 110.199 108.505) (end 108.924 108.505) (width 0.25) (layer F.Cu) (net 6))
 (segment (start 106.95 101.2345) (end 108.924 103.2085) (width 0.25) (layer B.Cu) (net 6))
 (segment (start 108.924 103.2085) (end 108.924 108.505) (width 0.25) (layer B.Cu) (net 6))
 (segment (start 105.918 105.041) (end 105.918 102.2665) (width 0.25) (layer F.Cu) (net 6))
 (segment (start 105.918 102.2665) (end 106.95 101.2345) (width 0.25) (layer F.Cu) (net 6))
 (segment (start 110.859 113.538) (end 111.6341 113.538) (width 0.25) (layer F.Cu) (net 6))
 (segment (start 103.505 121.92) (end 103.505 123.2951) (width 0.25) (layer F.Cu) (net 6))
 (segment (start 107.95 123.825) (end 104.0349 123.825) (width 0.25) (layer F.Cu) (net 6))
 (segment (start 104.0349 123.825) (end 103.505 123.2951) (width 0.25) (layer F.Cu) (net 6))
 (via (at 111.8195 118.5589) (size 0.6) (layers F.Cu B.Cu) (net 6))
 (via (at 120.022 123.033) (size 0.6) (layers F.Cu B.Cu) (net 6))
 (via (at 123.1415 121.2444) (size 0.6) (layers F.Cu B.Cu) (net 6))
 (via (at 106.1785 120.9445) (size 0.6) (layers F.Cu B.Cu) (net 6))
 (via (at 108.924 108.505) (size 0.6) (layers F.Cu B.Cu) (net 6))
 (via (at 106.95 101.2345) (size 0.6) (layers F.Cu B.Cu) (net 6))
 (segment (start 105.2 108.8) (end 101.2 108.8) (width 0.25) (layer B.Cu) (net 6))
 (segment (start 106.1 108.8) (end 106.1785 108.7215) (width 0.25) (layer B.Cu) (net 6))
 (segment (start 105.2 108.8) (end 106.1 108.8) (width 0.25) (layer B.Cu) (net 6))
 (segment (start 106.1785 108.7215) (end 106.1785 120.9445) (width 0.25) (layer B.Cu) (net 6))
 (segment (start 106.1785 102.006) (end 106.1785 108.7215) (width 0.25) (layer B.Cu) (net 6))
 (segment (start 103.505 116.84) (end 106.311 116.84) (width 0.5) (layer F.Cu) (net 20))
 (segment (start 119.177 107.235) (end 120.316 107.235) (width 0.3) (layer F.Cu) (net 2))
 (segment (start 120.316 107.235) (end 121.351 108.27) (width 0.3) (layer F.Cu) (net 2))
 (segment (start 121.351 108.27) (end 121.793 108.27) (width 0.3) (layer F.Cu) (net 2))
 (segment (start 110.3715 103.425) (end 110.372 103.425) (width 0.3) (layer F.Cu) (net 10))
 (segment (start 121.793 105.095) (end 121.793 104.267) (width 0.3) (layer F.Cu) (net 10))
 (segment (start 121.793 104.267) (end 120.562 103.036) (width 0.3) (layer F.Cu) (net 10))
 (segment (start 120.562 103.036) (end 120.562 101.131) (width 0.3) (layer F.Cu) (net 10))
 (segment (start 120.562 101.131) (end 120.015 100.584) (width 0.3) (layer F.Cu) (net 10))
 (segment (start 120.015 100.584) (end 109.347 100.584) (width 0.3) (layer F.Cu) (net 10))
 (segment (start 109.347 100.584) (end 108.966 100.965) (width 0.3) (layer F.Cu) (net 10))
 (segment (start 108.966 100.965) (end 108.966 103.124) (width 0.3) (layer F.Cu) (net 10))
 (segment (start 108.966 103.124) (end 109.267 103.425) (width 0.3) (layer F.Cu) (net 10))
 (segment (start 109.267 103.425) (end 110.3715 103.425) (width 0.3) (layer F.Cu) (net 10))
 (segment (start 123.825 108.27) (end 123.825 109.22) (width 0.3) (layer F.Cu) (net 1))
 (segment (start 123.825 109.22) (end 120.777 109.22) (width 0.3) (layer F.Cu) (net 1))
 (segment (start 120.777 109.22) (end 120.062 108.505) (width 0.3) (layer F.Cu) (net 1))
 (segment (start 120.062 108.505) (end 119.177 108.505) (width 0.3) (layer F.Cu) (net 1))
 (segment (start 123.825 108.27) (end 123.825 107.569) (width 0.3) (layer F.Cu) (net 1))
 (segment (start 123.825 107.569) (end 123.251 106.995) (width 0.3) (layer F.Cu) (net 1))
 (segment (start 123.251 106.995) (end 121.793 106.995) (width 0.3) (layer F.Cu) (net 1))
 (segment (start 101.41 114.488) (end 101.41 115.126) (width 0.35) (layer F.Cu) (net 21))
 (segment (start 101.41 115.126) (end 100.965 115.57) (width 0.35) (layer F.Cu) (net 21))
 (segment (start 100.965 115.57) (end 100.965 118.999) (width 0.35) (layer F.Cu) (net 21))
 (segment (start 100.965 118.999) (end 101.346 119.38) (width 0.35) (layer F.Cu) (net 21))
 (segment (start 101.346 119.38) (end 103.505 119.38) (width 0.35) (layer F.Cu) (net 21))
 (segment (start 102.364 108.752) (end 102.362 108.755) (width 0.35) (layer F.Cu) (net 12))
 (segment (start 102.364 106.87) (end 102.364 108.752) (width 0.3) (layer F.Cu) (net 12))
 (segment (start 102.364 106.87) (end 100.965 106.87) (width 0.3) (layer F.Cu) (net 12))
 (segment (start 111.059 120.396) (end 111.059 121.412) (width 0.35) (layer F.Cu) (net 15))
 (segment (start 111.059 119.464) (end 111.059 120.396) (width 0.35) (layer F.Cu) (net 15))
 (segment (start 111.059 120.396) (end 114.046 120.396) (width 0.3) (layer F.Cu) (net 15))
 (segment (start 114.046 120.396) (end 114.3 120.142) (width 0.3) (layer F.Cu) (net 15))
 (segment (start 114.3 120.142) (end 114.3 116.586) (width 0.3) (layer F.Cu) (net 15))
 (segment (start 114.3 116.586) (end 114.046 116.332) (width 0.3) (layer F.Cu) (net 15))
 (segment (start 114.046 116.332) (end 113.284 116.332) (width 0.3) (layer F.Cu) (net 15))
 (segment (start 113.284 116.332) (end 113.096 116.144) (width 0.3) (layer F.Cu) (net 15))
 (segment (start 113.096 116.144) (end 113.096 115.273) (width 0.3) (layer F.Cu) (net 15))
 (segment (start 101.412 112.586) (end 101.41 112.588) (width 0.35) (layer F.Cu) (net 13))
 (segment (start 101.412 110.955) (end 101.412 112.586) (width 0.3) (layer F.Cu) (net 13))
 (segment (start 122.004 124.206) (end 122.004 121.328) (width 0.35) (layer F.Cu) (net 18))
 (segment (start 122.004 121.328) (end 123.888 119.444) (width 0.35) (layer F.Cu) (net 18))
 (segment (start 123.888 119.444) (end 125.794 119.444) (width 0.35) (layer F.Cu) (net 18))
 (segment (start 125.794 119.444) (end 126.365 118.872) (width 0.35) (layer F.Cu) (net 18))
 (segment (start 126.365 118.872) (end 126.365 115.377) (width 0.35) (layer F.Cu) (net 18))
 (segment (start 119.761 113.538) (end 119.761 114.765) (width 0.35) (layer F.Cu) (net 19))
 (segment (start 119.761 114.765) (end 119.804 114.808) (width 0.35) (layer F.Cu) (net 19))
 (segment (start 107.696 103.759) (end 107.696 102.809) (width 0.3) (layer F.Cu) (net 19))
 (segment (start 119.761 113.538) (end 119.761 112.903) (width 0.3) (layer B.Cu) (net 19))
 (segment (start 119.761 112.903) (end 119.126 112.268) (width 0.3) (layer B.Cu) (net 19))
 (segment (start 119.126 112.268) (end 109.093 112.268) (width 0.3) (layer B.Cu) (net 19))
 (segment (start 109.093 112.268) (end 107.696 110.871) (width 0.3) (layer B.Cu) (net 19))
 (segment (start 107.696 110.871) (end 107.696 103.759) (width 0.3) (layer B.Cu) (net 19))
 (via (at 107.696 103.759) (size 0.6) (layers F.Cu B.Cu) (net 19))
 (via (at 119.761 113.538) (size 0.6) (layers F.Cu B.Cu) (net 19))
 (segment (start 110.199 104.695) (end 107.71 104.695) (width 0.3) (layer F.Cu) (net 9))
 (segment (start 107.71 104.695) (end 107.696 104.709) (width 0.35) (layer F.Cu) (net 9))
 (segment (start 111.059 117.264) (end 112.93 117.264) (width 0.3) (layer F.Cu) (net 16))
 (segment (start 112.93 117.264) (end 113.03 117.364) (width 0.3) (layer F.Cu) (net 16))
 (segment (start 103.312 109.6602) (end 103.31 109.6622) (width 0.25) (layer F.Cu) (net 11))
 (segment (start 103.31 109.6622) (end 103.31 109.855) (width 0.25) (layer F.Cu) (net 11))
 (segment (start 103.312 109.6602) (end 103.312 108.755) (width 0.3) (layer F.Cu) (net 11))
 (segment (start 103.312 109.852) (end 103.312 109.6602) (width 0.3) (layer F.Cu) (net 11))
 (segment (start 103.31 109.855) (end 102.362 109.855) (width 0.3) (layer F.Cu) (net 11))
 (segment (start 102.362 109.855) (end 102.362 111.76) (width 0.3) (layer F.Cu) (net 11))
 (segment (start 102.362 111.76) (end 103.19 112.588) (width 0.3) (layer F.Cu) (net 11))
 (segment (start 103.19 112.588) (end 103.19 113.538) (width 0.3) (layer F.Cu) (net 11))
 (segment (start 118.491 117.257) (end 124.884 117.257) (width 0.3) (layer F.Cu) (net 22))
 (segment (start 116.924 117.257) (end 118.491 117.257) (width 0.3) (layer F.Cu) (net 22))
 (segment (start 114.996 113.073) (end 114.996 114.173) (width 0.3) (layer F.Cu) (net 22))
 (segment (start 114.996 114.173) (end 117.983 114.173) (width 0.3) (layer F.Cu) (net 22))
 (segment (start 117.983 114.173) (end 118.491 114.681) (width 0.3) (layer F.Cu) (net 22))
 (segment (start 118.491 114.681) (end 118.491 117.257) (width 0.3) (layer F.Cu) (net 22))
 (segment (start 107.696 108.093) (end 107.68 108.093) (width 0.35) (layer F.Cu) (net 7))
 (segment (start 107.696 108.093) (end 107.68 108.093) (width 0.35) (layer F.Cu) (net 7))
 (segment (start 110.199 107.235) (end 108.554 107.235) (width 0.35) (layer F.Cu) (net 7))
 (segment (start 108.554 107.235) (end 107.696 108.093) (width 0.35) (layer F.Cu) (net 7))
 (segment (start 107.696 111.636) (end 106.81 111.636) (width 0.35) (layer F.Cu) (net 7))
 (segment (start 106.81 111.636) (end 106.426 111.252) (width 0.35) (layer F.Cu) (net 7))
 (segment (start 106.426 111.252) (end 106.426 108.458) (width 0.35) (layer F.Cu) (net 7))
 (segment (start 106.426 108.458) (end 106.791 108.093) (width 0.35) (layer F.Cu) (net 7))
 (segment (start 106.791 108.093) (end 107.68 108.093) (width 0.35) (layer F.Cu) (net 7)))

